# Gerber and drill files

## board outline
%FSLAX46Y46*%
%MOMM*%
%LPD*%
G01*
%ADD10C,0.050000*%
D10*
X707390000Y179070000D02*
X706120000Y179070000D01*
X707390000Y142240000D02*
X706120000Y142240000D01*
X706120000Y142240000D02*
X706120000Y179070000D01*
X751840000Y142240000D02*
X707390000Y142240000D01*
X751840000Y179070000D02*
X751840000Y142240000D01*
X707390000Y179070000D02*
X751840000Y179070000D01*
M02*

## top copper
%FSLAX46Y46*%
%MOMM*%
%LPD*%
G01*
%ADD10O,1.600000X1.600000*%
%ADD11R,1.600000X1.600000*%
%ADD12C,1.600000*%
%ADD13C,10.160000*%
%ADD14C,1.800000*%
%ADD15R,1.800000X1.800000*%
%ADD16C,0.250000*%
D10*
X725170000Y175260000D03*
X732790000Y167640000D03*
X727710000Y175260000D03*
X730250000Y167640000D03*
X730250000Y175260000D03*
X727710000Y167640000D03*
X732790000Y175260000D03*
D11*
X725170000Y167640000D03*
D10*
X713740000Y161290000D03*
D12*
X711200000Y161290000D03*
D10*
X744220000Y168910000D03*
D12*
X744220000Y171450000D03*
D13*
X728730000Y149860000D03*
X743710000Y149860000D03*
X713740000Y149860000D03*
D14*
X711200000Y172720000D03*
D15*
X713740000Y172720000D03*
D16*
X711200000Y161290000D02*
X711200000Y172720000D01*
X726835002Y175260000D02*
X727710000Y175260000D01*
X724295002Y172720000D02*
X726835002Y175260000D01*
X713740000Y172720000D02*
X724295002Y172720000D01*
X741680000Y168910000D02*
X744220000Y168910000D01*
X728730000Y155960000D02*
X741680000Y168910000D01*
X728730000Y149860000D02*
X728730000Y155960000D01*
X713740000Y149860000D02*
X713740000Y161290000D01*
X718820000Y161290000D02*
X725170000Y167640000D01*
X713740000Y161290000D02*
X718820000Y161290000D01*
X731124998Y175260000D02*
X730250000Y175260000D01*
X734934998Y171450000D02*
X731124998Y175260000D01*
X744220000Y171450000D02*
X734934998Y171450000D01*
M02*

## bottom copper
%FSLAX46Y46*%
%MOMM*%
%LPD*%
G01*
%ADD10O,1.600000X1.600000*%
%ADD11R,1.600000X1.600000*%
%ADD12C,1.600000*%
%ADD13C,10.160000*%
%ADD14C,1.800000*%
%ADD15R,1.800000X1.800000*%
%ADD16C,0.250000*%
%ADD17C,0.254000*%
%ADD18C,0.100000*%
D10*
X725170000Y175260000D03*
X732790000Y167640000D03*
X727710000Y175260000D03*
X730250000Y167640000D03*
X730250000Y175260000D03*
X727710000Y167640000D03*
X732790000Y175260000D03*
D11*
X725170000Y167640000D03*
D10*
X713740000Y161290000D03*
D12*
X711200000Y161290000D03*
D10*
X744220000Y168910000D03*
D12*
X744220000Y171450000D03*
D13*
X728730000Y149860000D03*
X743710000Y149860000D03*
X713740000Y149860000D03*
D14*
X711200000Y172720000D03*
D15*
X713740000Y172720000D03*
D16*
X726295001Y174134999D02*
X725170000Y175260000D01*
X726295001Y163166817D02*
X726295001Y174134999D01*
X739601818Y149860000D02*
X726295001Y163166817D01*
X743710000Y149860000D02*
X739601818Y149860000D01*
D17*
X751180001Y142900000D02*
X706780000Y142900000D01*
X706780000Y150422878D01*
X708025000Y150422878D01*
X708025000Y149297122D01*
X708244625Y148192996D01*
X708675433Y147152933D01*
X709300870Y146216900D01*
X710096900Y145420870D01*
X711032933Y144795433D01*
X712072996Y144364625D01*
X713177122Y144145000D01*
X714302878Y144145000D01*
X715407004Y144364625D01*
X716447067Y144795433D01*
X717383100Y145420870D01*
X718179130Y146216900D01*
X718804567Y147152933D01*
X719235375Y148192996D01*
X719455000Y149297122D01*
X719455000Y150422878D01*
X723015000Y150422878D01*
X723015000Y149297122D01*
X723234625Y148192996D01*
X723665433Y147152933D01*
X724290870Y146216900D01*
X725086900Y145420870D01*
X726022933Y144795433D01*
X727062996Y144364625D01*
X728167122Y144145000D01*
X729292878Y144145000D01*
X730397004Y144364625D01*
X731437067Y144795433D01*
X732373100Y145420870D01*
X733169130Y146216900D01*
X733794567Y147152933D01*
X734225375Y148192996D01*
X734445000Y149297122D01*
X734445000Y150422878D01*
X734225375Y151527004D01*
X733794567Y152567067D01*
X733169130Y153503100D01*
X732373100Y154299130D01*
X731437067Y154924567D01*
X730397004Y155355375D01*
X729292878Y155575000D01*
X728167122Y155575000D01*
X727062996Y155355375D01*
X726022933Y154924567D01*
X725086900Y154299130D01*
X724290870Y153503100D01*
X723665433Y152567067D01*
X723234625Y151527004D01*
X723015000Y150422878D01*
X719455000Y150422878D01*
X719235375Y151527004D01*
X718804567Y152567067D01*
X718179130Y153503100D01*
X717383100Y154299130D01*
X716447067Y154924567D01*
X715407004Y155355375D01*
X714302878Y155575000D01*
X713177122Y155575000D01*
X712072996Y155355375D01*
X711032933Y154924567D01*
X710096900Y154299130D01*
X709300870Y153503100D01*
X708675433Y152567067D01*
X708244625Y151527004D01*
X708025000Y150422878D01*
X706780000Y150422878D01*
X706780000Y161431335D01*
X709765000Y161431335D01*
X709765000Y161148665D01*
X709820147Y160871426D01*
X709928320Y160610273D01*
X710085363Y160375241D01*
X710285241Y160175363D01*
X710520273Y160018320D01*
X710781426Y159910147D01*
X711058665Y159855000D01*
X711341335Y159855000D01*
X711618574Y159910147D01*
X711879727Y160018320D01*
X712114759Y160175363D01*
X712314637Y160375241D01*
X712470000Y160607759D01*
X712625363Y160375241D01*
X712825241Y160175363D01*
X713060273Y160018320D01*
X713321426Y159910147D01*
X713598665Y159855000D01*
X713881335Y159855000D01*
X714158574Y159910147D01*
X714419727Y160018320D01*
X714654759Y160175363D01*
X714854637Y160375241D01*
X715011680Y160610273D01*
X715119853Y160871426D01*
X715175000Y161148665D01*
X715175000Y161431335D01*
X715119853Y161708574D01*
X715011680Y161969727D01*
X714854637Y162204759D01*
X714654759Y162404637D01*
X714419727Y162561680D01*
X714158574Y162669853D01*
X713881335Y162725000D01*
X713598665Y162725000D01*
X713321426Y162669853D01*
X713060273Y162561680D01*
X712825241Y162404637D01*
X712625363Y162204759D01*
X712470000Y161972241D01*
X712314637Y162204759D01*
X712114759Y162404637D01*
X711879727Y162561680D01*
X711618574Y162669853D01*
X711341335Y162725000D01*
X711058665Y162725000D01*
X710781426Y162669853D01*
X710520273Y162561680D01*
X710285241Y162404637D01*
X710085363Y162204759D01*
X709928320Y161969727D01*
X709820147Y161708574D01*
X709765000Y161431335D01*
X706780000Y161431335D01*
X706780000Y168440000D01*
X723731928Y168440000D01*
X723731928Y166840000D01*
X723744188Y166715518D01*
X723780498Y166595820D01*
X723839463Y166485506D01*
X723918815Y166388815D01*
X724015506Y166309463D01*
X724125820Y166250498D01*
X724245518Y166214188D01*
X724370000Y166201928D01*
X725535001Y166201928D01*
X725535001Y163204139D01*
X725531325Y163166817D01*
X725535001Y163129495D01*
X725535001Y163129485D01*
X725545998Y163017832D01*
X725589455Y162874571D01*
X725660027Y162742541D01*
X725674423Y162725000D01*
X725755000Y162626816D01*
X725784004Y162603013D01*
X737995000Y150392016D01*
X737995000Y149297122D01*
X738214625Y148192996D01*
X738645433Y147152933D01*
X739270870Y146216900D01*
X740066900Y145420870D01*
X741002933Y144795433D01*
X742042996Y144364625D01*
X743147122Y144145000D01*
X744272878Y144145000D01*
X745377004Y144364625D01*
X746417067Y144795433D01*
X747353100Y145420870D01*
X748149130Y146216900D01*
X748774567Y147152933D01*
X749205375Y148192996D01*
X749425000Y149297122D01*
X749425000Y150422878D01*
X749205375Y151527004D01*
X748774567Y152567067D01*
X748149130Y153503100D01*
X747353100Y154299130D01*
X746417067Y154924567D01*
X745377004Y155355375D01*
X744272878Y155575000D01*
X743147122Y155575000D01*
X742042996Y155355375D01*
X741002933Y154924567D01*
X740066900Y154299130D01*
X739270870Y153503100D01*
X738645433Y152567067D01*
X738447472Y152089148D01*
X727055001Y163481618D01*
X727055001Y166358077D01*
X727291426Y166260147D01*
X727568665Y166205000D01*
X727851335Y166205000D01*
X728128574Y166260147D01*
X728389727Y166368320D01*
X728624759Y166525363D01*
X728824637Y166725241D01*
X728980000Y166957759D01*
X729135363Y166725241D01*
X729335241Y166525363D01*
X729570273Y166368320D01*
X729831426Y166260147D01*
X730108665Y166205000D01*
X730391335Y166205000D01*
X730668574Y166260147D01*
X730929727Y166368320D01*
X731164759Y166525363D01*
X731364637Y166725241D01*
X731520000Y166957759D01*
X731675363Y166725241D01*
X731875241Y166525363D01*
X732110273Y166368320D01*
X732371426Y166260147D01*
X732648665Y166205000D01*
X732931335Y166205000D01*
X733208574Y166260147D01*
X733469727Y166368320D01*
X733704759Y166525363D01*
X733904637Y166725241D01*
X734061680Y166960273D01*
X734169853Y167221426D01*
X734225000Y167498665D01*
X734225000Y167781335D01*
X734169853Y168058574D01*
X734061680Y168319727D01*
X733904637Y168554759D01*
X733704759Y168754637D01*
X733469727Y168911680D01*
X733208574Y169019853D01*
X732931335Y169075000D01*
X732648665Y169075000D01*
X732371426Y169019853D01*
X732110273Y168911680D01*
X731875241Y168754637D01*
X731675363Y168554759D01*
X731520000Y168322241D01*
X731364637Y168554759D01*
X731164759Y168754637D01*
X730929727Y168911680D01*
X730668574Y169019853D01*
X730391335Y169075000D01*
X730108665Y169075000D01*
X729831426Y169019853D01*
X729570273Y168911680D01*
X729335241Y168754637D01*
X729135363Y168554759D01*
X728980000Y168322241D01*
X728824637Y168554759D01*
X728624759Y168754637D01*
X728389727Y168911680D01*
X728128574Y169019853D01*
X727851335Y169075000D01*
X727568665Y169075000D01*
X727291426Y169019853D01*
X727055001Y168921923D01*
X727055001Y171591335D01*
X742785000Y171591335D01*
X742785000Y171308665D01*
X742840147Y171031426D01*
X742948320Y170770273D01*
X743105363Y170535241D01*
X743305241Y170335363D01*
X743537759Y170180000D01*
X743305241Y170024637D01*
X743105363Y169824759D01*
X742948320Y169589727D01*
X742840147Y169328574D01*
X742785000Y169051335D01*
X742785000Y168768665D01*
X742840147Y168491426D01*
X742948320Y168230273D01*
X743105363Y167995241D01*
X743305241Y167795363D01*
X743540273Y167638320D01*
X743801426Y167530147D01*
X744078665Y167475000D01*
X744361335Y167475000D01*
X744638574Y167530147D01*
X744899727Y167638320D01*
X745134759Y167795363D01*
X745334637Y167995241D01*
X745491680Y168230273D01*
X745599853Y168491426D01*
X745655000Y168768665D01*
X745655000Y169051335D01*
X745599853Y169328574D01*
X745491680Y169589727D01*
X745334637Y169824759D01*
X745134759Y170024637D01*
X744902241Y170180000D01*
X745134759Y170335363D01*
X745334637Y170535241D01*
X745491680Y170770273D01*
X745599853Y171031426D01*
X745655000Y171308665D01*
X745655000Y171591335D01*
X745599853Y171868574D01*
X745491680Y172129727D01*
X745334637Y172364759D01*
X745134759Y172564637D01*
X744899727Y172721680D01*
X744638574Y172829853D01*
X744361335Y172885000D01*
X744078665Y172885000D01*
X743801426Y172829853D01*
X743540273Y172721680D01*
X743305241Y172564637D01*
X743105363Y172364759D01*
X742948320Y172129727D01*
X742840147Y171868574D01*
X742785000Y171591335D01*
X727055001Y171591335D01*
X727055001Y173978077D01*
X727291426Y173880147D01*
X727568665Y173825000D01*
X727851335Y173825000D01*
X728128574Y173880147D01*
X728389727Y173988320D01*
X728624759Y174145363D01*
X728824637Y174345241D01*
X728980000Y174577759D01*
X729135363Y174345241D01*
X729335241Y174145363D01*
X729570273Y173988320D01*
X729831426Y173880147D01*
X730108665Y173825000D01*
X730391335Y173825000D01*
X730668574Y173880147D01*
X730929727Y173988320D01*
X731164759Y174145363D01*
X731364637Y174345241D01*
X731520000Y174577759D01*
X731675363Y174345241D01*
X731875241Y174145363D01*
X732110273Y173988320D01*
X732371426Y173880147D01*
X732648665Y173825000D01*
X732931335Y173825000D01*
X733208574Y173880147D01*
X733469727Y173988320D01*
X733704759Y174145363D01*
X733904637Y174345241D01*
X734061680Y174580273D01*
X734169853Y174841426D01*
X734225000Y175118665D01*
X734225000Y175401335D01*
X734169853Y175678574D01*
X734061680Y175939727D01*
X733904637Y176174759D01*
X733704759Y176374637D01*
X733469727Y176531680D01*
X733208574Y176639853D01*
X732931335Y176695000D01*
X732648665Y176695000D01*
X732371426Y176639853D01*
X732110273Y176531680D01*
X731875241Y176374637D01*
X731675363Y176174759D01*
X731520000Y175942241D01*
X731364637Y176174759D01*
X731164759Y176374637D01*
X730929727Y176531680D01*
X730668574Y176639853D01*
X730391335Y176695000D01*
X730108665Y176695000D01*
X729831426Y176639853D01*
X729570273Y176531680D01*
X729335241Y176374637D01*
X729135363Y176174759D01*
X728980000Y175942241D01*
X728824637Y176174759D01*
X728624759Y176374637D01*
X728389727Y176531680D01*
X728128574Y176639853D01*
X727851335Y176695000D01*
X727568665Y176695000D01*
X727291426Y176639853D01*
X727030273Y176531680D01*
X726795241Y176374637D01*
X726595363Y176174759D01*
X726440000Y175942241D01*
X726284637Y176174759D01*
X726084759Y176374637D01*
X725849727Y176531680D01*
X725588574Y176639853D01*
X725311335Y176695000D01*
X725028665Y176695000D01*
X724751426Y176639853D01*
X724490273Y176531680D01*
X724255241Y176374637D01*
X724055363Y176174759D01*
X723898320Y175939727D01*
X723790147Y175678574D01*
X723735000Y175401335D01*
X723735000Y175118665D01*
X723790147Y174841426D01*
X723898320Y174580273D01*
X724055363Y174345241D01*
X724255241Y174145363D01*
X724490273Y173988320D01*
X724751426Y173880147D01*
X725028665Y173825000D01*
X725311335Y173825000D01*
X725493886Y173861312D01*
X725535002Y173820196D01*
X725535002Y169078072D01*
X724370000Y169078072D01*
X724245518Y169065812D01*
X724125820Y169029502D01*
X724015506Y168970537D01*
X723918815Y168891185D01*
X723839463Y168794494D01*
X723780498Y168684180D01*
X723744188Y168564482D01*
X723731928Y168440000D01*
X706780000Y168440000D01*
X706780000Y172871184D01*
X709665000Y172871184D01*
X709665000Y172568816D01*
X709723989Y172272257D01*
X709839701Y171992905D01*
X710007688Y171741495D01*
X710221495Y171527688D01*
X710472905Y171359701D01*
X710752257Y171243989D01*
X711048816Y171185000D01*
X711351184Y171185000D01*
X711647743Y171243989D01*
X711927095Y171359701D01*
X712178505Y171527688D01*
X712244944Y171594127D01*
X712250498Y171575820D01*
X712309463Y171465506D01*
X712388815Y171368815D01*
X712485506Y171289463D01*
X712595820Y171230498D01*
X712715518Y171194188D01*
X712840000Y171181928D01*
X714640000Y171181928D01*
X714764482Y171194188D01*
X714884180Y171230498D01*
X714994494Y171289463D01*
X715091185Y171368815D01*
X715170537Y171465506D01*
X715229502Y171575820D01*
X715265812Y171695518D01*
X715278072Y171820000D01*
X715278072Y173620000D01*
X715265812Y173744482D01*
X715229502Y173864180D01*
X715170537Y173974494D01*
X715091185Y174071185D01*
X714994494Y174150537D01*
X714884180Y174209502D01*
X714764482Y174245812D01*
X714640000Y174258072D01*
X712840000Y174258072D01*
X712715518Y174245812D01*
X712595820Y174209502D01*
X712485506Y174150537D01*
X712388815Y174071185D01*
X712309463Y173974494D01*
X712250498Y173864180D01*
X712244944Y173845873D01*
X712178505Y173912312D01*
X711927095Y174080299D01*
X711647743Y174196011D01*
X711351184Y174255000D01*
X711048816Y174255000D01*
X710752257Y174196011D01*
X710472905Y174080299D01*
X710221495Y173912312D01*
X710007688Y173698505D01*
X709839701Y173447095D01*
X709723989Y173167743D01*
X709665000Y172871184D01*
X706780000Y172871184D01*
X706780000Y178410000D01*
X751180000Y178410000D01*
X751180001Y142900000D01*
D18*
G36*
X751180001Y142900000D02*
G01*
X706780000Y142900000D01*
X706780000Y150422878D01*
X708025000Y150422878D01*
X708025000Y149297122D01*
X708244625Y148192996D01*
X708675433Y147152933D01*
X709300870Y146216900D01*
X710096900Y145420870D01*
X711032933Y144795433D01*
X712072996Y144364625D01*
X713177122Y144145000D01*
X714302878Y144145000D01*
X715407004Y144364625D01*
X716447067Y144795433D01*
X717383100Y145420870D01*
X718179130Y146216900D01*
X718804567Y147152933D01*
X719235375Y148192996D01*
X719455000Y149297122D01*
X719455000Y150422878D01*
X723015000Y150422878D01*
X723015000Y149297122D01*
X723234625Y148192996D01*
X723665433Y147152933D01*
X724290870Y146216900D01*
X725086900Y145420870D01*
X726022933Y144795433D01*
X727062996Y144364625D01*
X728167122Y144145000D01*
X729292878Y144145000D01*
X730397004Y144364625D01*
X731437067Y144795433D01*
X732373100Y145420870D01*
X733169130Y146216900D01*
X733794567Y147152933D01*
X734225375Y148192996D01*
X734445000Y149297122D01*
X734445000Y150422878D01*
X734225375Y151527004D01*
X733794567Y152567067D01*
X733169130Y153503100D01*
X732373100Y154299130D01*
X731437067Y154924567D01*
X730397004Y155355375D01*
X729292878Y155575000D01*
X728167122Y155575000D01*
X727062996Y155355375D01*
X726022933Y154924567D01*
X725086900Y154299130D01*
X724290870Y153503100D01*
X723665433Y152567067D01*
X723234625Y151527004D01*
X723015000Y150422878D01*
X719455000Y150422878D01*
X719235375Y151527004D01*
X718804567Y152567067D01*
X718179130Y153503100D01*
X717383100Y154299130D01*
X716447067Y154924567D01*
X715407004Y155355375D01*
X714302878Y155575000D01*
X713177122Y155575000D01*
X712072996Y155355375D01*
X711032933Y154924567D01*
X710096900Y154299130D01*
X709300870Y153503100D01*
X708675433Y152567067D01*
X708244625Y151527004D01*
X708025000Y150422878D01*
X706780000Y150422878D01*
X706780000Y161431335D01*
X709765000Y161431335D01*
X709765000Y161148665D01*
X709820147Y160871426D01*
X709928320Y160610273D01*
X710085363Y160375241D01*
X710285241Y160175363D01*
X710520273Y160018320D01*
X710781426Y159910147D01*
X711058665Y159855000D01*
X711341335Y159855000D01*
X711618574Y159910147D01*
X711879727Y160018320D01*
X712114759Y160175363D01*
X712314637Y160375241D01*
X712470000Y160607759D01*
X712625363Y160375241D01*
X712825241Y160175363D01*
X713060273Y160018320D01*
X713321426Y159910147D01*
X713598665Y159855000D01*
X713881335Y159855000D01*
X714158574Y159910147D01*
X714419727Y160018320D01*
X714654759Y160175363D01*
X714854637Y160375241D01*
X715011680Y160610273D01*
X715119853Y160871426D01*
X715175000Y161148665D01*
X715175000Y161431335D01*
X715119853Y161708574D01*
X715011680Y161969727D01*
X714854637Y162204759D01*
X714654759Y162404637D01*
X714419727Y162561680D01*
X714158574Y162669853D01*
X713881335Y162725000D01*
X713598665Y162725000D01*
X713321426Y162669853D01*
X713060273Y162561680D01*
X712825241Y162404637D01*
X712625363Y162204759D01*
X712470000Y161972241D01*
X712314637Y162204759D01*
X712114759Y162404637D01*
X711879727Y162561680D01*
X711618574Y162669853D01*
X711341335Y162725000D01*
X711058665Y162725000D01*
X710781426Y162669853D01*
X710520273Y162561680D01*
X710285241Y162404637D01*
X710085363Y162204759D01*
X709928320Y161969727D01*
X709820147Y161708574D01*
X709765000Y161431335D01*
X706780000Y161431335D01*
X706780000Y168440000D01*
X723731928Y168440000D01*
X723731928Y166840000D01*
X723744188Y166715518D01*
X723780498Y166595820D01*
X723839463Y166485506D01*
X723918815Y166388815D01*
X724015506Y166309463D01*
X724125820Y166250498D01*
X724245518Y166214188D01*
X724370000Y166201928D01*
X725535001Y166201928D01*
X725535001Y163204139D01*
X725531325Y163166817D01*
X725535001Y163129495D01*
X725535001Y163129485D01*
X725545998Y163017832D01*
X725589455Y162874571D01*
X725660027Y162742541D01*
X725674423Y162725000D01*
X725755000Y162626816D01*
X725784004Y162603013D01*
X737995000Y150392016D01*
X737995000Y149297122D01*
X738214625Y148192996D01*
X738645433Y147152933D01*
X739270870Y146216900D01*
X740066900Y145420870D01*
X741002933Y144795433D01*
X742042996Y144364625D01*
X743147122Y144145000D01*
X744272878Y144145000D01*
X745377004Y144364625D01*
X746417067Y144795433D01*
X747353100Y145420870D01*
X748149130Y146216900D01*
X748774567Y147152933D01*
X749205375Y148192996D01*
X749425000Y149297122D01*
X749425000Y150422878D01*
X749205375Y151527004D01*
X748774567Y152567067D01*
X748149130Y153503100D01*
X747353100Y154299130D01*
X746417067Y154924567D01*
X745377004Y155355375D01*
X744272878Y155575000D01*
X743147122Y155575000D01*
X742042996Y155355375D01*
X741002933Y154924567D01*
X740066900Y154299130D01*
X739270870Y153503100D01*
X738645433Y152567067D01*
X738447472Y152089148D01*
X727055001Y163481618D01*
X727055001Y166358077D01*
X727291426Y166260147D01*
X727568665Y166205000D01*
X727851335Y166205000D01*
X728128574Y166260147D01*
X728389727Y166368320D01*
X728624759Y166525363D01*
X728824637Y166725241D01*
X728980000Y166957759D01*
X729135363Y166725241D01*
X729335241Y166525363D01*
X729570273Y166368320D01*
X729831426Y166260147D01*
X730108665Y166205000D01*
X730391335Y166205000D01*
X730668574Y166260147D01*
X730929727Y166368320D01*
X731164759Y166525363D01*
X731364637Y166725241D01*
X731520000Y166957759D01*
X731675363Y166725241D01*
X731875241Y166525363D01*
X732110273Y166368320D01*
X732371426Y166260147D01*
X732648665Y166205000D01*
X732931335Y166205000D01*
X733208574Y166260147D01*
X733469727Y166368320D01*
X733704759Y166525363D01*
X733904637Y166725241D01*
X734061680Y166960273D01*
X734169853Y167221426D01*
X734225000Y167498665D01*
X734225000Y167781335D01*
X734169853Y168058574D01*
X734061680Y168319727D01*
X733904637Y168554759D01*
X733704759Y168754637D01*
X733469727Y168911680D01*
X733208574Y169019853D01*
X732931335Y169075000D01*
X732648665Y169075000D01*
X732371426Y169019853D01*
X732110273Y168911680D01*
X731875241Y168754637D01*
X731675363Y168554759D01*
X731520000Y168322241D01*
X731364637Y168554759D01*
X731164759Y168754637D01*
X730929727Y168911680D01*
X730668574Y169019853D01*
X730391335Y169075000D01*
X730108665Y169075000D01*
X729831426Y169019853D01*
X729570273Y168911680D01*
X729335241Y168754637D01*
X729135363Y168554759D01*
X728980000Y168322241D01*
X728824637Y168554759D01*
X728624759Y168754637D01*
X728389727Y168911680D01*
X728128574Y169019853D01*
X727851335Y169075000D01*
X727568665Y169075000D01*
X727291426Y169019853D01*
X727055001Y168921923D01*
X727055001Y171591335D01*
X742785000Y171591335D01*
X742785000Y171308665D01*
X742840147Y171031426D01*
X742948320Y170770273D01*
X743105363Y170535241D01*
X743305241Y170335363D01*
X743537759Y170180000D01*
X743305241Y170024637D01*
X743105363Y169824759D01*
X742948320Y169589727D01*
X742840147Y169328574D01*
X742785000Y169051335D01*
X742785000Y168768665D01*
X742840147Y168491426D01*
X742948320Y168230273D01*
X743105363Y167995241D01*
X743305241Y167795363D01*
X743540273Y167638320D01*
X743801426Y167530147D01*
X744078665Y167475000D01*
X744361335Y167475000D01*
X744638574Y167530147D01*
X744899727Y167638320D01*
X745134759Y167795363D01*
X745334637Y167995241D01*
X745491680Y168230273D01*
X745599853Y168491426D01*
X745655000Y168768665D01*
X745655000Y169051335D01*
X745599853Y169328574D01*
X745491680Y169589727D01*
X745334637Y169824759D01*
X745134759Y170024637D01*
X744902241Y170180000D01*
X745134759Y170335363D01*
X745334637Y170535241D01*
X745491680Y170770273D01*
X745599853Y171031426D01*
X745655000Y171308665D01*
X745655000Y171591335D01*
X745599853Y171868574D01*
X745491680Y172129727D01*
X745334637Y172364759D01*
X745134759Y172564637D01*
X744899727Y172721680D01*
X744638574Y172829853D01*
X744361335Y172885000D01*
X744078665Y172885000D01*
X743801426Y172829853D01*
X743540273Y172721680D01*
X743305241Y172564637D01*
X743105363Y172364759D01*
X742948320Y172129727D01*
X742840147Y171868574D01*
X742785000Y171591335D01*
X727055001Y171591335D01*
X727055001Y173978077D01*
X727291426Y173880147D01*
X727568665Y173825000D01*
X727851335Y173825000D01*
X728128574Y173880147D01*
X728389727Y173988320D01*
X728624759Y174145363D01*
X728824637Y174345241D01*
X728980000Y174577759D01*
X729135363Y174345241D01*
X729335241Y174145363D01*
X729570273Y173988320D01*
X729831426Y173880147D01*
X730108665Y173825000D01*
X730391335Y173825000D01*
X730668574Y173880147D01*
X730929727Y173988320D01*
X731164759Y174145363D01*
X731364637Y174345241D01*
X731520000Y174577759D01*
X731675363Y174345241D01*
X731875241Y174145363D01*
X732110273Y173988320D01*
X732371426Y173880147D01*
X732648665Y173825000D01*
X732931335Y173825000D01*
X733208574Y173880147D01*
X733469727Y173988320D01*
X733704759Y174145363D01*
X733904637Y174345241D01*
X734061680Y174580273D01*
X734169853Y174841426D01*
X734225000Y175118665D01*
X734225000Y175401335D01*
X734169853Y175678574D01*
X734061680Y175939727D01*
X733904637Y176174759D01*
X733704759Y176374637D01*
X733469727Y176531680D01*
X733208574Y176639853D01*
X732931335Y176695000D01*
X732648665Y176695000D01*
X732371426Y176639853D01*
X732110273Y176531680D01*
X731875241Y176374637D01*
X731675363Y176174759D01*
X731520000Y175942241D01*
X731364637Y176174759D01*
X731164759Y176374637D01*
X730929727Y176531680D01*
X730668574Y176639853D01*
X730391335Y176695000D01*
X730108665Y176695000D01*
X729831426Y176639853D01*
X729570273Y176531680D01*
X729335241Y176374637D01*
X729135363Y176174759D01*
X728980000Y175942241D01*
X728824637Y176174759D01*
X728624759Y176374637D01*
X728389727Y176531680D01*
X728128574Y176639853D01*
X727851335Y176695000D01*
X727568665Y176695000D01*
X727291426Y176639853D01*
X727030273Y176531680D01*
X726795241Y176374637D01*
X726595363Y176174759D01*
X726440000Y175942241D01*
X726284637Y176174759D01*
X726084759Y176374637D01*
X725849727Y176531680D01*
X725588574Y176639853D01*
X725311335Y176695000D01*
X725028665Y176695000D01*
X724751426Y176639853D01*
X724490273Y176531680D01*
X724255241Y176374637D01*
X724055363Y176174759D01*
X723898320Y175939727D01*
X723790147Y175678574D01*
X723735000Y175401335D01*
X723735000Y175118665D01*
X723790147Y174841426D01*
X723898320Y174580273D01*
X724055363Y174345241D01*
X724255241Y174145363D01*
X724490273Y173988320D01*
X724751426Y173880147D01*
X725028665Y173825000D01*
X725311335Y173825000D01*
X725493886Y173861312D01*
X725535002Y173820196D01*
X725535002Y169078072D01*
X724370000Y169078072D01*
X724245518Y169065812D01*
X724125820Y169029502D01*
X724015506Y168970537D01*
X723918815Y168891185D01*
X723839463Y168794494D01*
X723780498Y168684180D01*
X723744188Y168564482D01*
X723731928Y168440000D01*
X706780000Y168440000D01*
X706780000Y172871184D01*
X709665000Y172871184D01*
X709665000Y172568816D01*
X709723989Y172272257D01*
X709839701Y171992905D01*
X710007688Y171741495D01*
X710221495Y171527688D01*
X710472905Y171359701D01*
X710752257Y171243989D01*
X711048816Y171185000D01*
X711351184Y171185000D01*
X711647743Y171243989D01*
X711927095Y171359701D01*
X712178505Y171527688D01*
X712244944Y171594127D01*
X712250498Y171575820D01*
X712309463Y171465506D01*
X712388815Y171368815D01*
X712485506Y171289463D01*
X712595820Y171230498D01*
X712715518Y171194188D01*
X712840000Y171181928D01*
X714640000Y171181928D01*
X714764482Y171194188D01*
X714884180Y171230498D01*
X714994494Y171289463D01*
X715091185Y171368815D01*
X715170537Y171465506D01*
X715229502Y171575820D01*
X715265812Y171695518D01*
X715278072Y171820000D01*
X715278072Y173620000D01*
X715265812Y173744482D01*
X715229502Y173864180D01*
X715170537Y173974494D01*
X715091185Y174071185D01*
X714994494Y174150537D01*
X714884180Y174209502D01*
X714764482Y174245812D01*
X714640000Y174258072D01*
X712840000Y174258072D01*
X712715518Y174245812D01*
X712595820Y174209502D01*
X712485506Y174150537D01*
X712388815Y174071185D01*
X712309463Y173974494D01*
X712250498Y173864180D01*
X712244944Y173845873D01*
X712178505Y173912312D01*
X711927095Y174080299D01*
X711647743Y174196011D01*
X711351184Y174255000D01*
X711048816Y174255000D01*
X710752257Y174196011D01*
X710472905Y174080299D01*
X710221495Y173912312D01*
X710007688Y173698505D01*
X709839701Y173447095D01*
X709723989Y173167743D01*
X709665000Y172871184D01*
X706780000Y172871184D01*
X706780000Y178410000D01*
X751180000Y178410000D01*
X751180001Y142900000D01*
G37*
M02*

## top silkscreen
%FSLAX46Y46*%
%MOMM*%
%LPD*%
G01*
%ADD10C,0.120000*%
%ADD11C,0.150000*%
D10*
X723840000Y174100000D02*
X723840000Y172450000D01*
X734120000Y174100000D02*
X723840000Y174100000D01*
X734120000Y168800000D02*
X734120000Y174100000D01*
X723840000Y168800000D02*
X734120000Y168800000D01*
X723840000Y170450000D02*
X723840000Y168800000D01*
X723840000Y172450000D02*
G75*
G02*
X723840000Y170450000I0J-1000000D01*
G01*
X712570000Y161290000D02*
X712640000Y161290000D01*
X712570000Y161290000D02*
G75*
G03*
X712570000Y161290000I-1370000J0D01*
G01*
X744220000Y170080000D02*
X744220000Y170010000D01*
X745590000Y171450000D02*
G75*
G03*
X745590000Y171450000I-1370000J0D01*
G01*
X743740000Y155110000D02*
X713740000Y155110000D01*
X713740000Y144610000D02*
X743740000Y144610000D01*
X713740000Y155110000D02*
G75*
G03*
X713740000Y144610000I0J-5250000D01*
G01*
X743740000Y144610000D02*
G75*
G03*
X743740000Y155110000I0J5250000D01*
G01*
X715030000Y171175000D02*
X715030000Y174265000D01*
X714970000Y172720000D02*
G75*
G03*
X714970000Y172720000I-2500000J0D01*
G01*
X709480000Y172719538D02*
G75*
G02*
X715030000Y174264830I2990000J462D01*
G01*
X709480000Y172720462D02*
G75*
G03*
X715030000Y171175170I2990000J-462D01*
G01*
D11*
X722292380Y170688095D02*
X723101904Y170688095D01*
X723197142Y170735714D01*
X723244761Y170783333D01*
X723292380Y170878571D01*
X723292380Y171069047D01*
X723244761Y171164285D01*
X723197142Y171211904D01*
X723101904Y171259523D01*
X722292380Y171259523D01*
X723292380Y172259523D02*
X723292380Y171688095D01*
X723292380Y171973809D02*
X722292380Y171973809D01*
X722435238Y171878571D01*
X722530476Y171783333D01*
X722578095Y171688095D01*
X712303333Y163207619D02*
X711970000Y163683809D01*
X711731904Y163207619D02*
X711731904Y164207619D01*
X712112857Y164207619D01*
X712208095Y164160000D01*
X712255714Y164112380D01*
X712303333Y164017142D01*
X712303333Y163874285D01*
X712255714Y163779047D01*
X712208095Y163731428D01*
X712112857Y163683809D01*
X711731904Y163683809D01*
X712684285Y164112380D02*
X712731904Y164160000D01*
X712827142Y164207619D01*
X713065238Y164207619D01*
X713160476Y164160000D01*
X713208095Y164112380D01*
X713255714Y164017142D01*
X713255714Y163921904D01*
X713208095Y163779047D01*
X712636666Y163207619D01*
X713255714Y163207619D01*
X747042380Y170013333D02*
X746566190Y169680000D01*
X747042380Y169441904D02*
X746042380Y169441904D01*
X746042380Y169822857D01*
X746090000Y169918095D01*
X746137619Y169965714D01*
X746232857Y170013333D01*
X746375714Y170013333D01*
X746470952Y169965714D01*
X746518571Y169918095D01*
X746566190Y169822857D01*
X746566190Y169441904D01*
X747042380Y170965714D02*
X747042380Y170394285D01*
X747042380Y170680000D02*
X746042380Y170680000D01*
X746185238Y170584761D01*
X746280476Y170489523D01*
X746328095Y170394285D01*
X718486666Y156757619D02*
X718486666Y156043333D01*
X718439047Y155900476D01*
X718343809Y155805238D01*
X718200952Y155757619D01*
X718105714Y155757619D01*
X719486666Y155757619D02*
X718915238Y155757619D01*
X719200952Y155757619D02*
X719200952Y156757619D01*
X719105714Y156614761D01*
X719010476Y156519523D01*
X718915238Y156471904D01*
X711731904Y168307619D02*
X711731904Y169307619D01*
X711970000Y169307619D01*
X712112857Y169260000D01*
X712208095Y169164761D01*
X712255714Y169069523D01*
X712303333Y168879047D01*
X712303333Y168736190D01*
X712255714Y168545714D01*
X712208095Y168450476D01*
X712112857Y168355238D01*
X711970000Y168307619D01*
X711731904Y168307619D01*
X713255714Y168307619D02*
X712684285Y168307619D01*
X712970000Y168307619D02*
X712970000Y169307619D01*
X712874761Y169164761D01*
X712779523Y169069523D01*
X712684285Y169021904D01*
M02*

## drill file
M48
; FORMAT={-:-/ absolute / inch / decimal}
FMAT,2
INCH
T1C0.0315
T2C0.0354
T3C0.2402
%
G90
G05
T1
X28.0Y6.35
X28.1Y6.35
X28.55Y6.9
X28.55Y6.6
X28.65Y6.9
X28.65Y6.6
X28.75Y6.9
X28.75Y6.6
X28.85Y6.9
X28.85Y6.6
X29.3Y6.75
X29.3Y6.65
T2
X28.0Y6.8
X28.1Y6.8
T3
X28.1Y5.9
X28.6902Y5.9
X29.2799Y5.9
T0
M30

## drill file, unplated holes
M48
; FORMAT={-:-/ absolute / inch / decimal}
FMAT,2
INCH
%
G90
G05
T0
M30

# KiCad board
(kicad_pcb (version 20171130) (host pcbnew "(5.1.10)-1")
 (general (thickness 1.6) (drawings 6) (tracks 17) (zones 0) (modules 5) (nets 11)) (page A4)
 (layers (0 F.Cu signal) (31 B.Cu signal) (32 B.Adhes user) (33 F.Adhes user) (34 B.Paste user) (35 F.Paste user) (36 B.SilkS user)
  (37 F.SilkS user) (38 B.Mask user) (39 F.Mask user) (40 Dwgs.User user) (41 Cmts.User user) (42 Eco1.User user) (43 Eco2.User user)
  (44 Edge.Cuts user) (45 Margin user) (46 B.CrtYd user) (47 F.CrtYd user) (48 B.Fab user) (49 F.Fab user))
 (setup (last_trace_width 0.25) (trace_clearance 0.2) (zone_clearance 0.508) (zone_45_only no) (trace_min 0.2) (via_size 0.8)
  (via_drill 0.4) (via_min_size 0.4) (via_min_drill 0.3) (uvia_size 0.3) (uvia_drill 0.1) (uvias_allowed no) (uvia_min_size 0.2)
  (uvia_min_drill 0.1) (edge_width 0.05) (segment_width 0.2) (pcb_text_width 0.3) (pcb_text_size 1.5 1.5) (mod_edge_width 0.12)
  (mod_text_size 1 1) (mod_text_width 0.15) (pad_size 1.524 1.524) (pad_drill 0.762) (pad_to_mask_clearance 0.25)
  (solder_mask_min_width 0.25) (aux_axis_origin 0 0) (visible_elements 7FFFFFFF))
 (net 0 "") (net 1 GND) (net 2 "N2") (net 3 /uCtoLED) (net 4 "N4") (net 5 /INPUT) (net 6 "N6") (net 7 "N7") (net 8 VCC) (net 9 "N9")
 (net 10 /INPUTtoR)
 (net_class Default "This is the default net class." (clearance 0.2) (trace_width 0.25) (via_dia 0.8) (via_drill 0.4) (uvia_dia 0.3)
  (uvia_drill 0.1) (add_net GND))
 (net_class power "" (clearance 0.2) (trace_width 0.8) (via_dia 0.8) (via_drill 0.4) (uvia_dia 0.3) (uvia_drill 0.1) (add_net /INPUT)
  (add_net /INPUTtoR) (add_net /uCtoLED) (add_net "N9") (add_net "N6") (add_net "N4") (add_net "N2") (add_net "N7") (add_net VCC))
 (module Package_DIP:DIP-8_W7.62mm (layer F.Cu) (at 725.17 -167.64 90)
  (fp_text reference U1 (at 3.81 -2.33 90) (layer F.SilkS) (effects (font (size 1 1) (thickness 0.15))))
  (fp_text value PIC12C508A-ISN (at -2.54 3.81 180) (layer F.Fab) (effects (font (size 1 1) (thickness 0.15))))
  (fp_line (start 6.46 -1.33) (end 4.81 -1.33) (layer F.SilkS) (width 0.12))
  (fp_line (start 6.46 8.95) (end 6.46 -1.33) (layer F.SilkS) (width 0.12))
  (fp_line (start 1.16 8.95) (end 6.46 8.95) (layer F.SilkS) (width 0.12))
  (fp_line (start 1.16 -1.33) (end 1.16 8.95) (layer F.SilkS) (width 0.12))
  (fp_line (start 2.81 -1.33) (end 1.16 -1.33) (layer F.SilkS) (width 0.12))
  (fp_arc (start 3.81 -1.33) (end 2.81 -1.33) (angle -180) (layer F.SilkS) (width 0.12))
  (pad 8 thru_hole oval (at 7.62 0 90) (size 1.6 1.6) (drill 0.8) (layers *.Cu *.Mask) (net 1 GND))
  (pad 4 thru_hole oval (at 0 7.62 90) (size 1.6 1.6) (drill 0.8) (layers *.Cu *.Mask) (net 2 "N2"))
  (pad 7 thru_hole oval (at 7.62 2.54 90) (size 1.6 1.6) (drill 0.8) (layers *.Cu *.Mask) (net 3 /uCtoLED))
  (pad 3 thru_hole oval (at 0 5.08 90) (size 1.6 1.6) (drill 0.8) (layers *.Cu *.Mask) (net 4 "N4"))
  (pad 6 thru_hole oval (at 7.62 5.08 90) (size 1.6 1.6) (drill 0.8) (layers *.Cu *.Mask) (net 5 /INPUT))
  (pad 2 thru_hole oval (at 0 2.54 90) (size 1.6 1.6) (drill 0.8) (layers *.Cu *.Mask) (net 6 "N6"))
  (pad 5 thru_hole oval (at 7.62 7.62 90) (size 1.6 1.6) (drill 0.8) (layers *.Cu *.Mask) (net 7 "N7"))
  (pad 1 thru_hole rect (at 0 0 90) (size 1.6 1.6) (drill 0.8) (layers *.Cu *.Mask) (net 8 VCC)))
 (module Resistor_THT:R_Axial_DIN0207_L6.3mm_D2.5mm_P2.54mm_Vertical (layer F.Cu) (at 711.2 -161.29)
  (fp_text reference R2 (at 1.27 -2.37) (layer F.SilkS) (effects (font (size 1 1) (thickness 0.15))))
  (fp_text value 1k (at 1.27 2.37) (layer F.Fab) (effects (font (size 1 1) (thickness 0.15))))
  (fp_line (start 1.37 0) (end 1.44 0) (layer F.SilkS) (width 0.12))
  (fp_circle (center 0 0) (end 1.37 0) (layer F.SilkS) (width 0.12))
  (pad 2 thru_hole oval (at 2.54 0) (size 1.6 1.6) (drill 0.8) (layers *.Cu *.Mask) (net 8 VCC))
  (pad 1 thru_hole circle (at 0 0) (size 1.6 1.6) (drill 0.8) (layers *.Cu *.Mask) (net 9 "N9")))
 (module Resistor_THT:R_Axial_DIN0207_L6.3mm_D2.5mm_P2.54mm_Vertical (layer F.Cu) (at 744.22 -171.45 270)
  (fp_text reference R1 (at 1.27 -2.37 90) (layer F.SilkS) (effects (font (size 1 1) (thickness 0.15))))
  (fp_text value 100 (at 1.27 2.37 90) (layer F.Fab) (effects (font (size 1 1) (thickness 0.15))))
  (fp_line (start 1.37 0) (end 1.44 0) (layer F.SilkS) (width 0.12))
  (fp_circle (center 0 0) (end 1.37 0) (layer F.SilkS) (width 0.12))
  (pad 2 thru_hole oval (at 2.54 0 270) (size 1.6 1.6) (drill 0.8) (layers *.Cu *.Mask) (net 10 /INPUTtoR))
  (pad 1 thru_hole circle (at 0 0 270) (size 1.6 1.6) (drill 0.8) (layers *.Cu *.Mask) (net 5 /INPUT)))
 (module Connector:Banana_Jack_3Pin (layer F.Cu) (at 713.74 -149.86)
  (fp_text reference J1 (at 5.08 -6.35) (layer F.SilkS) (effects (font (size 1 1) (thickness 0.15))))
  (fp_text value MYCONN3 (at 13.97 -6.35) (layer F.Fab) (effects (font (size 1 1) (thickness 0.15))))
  (fp_line (start 30 -5.25) (end 0 -5.25) (layer F.SilkS) (width 0.12))
  (fp_line (start 0 5.25) (end 30 5.25) (layer F.SilkS) (width 0.12))
  (fp_arc (start 0 0) (end 0 5.25) (angle 180) (layer F.SilkS) (width 0.12))
  (fp_arc (start 30 0) (end 30 -5.25) (angle 180) (layer F.SilkS) (width 0.12))
  (pad 2 thru_hole circle (at 14.99 0) (size 10.16 10.16) (drill 6.1) (layers *.Cu *.Mask) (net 10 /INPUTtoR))
  (pad 3 thru_hole circle (at 29.97 0) (size 10.16 10.16) (drill 6.1) (layers *.Cu *.Mask) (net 1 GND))
  (pad 1 thru_hole circle (at 0 0) (size 10.16 10.16) (drill 6.1) (layers *.Cu *.Mask) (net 8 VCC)))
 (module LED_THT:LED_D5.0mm (layer F.Cu) (at 713.74 -172.72 180)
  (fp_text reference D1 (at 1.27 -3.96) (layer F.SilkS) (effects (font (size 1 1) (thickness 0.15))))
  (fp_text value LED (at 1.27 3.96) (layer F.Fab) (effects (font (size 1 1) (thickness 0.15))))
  (fp_line (start -1.29 -1.545) (end -1.29 1.545) (layer F.SilkS) (width 0.12))
  (fp_circle (center 1.27 0) (end 3.77 0) (layer F.SilkS) (width 0.12))
  (fp_arc (start 1.27 0) (end -1.29 1.54483) (angle -148.9) (layer F.SilkS) (width 0.12))
  (fp_arc (start 1.27 0) (end -1.29 -1.54483) (angle 148.9) (layer F.SilkS) (width 0.12))
  (pad 2 thru_hole circle (at 2.54 0 180) (size 1.8 1.8) (drill 0.9) (layers *.Cu *.Mask) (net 9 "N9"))
  (pad 1 thru_hole rect (at 0 0 180) (size 1.8 1.8) (drill 0.9) (layers *.Cu *.Mask) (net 3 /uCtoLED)))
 (gr_line (start 707.39 -179.07) (end 706.12 -179.07) (layer Edge.Cuts) (width 0.05))
 (gr_line (start 707.39 -142.24) (end 706.12 -142.24) (layer Edge.Cuts) (width 0.05))
 (gr_line (start 706.12 -142.24) (end 706.12 -179.07) (layer Edge.Cuts) (width 0.05))
 (gr_line (start 751.84 -142.24) (end 707.39 -142.24) (layer Edge.Cuts) (width 0.05))
 (gr_line (start 751.84 -179.07) (end 751.84 -142.24) (layer Edge.Cuts) (width 0.05))
 (gr_line (start 707.39 -179.07) (end 751.84 -179.07) (layer Edge.Cuts) (width 0.05))
 (segment (start 711.2 -161.29) (end 711.2 -172.72) (width 0.25) (layer F.Cu) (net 9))
 (segment (start 726.835002 -175.26) (end 727.71 -175.26) (width 0.25) (layer F.Cu) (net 3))
 (segment (start 724.295002 -172.72) (end 726.835002 -175.26) (width 0.25) (layer F.Cu) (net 3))
 (segment (start 713.74 -172.72) (end 724.295002 -172.72) (width 0.25) (layer F.Cu) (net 3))
 (segment (start 741.68 -168.91) (end 744.22 -168.91) (width 0.25) (layer F.Cu) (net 10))
 (segment (start 728.73 -155.96) (end 741.68 -168.91) (width 0.25) (layer F.Cu) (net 10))
 (segment (start 728.73 -149.86) (end 728.73 -155.96) (width 0.25) (layer F.Cu) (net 10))
 (segment (start 726.295001 -174.134999) (end 725.17 -175.26) (width 0.25) (layer B.Cu) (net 1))
 (segment (start 726.295001 -163.166817) (end 726.295001 -174.134999) (width 0.25) (layer B.Cu) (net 1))
 (segment (start 739.601818 -149.86) (end 726.295001 -163.166817) (width 0.25) (layer B.Cu) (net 1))
 (segment (start 743.71 -149.86) (end 739.601818 -149.86) (width 0.25) (layer B.Cu) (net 1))
 (segment (start 713.74 -149.86) (end 713.74 -161.29) (width 0.25) (layer F.Cu) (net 8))
 (segment (start 718.82 -161.29) (end 725.17 -167.64) (width 0.25) (layer F.Cu) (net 8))
 (segment (start 713.74 -161.29) (end 718.82 -161.29) (width 0.25) (layer F.Cu) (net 8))
 (segment (start 731.124998 -175.26) (end 730.25 -175.26) (width 0.25) (layer F.Cu) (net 5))
 (segment (start 734.934998 -171.45) (end 731.124998 -175.26) (width 0.25) (layer F.Cu) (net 5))
 (segment (start 744.22 -171.45) (end 734.934998 -171.45) (width 0.25) (layer F.Cu) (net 5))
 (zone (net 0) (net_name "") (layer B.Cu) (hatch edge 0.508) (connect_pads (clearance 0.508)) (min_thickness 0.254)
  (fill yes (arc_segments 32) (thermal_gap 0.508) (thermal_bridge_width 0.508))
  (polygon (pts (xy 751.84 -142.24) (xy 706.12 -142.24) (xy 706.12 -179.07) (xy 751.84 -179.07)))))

